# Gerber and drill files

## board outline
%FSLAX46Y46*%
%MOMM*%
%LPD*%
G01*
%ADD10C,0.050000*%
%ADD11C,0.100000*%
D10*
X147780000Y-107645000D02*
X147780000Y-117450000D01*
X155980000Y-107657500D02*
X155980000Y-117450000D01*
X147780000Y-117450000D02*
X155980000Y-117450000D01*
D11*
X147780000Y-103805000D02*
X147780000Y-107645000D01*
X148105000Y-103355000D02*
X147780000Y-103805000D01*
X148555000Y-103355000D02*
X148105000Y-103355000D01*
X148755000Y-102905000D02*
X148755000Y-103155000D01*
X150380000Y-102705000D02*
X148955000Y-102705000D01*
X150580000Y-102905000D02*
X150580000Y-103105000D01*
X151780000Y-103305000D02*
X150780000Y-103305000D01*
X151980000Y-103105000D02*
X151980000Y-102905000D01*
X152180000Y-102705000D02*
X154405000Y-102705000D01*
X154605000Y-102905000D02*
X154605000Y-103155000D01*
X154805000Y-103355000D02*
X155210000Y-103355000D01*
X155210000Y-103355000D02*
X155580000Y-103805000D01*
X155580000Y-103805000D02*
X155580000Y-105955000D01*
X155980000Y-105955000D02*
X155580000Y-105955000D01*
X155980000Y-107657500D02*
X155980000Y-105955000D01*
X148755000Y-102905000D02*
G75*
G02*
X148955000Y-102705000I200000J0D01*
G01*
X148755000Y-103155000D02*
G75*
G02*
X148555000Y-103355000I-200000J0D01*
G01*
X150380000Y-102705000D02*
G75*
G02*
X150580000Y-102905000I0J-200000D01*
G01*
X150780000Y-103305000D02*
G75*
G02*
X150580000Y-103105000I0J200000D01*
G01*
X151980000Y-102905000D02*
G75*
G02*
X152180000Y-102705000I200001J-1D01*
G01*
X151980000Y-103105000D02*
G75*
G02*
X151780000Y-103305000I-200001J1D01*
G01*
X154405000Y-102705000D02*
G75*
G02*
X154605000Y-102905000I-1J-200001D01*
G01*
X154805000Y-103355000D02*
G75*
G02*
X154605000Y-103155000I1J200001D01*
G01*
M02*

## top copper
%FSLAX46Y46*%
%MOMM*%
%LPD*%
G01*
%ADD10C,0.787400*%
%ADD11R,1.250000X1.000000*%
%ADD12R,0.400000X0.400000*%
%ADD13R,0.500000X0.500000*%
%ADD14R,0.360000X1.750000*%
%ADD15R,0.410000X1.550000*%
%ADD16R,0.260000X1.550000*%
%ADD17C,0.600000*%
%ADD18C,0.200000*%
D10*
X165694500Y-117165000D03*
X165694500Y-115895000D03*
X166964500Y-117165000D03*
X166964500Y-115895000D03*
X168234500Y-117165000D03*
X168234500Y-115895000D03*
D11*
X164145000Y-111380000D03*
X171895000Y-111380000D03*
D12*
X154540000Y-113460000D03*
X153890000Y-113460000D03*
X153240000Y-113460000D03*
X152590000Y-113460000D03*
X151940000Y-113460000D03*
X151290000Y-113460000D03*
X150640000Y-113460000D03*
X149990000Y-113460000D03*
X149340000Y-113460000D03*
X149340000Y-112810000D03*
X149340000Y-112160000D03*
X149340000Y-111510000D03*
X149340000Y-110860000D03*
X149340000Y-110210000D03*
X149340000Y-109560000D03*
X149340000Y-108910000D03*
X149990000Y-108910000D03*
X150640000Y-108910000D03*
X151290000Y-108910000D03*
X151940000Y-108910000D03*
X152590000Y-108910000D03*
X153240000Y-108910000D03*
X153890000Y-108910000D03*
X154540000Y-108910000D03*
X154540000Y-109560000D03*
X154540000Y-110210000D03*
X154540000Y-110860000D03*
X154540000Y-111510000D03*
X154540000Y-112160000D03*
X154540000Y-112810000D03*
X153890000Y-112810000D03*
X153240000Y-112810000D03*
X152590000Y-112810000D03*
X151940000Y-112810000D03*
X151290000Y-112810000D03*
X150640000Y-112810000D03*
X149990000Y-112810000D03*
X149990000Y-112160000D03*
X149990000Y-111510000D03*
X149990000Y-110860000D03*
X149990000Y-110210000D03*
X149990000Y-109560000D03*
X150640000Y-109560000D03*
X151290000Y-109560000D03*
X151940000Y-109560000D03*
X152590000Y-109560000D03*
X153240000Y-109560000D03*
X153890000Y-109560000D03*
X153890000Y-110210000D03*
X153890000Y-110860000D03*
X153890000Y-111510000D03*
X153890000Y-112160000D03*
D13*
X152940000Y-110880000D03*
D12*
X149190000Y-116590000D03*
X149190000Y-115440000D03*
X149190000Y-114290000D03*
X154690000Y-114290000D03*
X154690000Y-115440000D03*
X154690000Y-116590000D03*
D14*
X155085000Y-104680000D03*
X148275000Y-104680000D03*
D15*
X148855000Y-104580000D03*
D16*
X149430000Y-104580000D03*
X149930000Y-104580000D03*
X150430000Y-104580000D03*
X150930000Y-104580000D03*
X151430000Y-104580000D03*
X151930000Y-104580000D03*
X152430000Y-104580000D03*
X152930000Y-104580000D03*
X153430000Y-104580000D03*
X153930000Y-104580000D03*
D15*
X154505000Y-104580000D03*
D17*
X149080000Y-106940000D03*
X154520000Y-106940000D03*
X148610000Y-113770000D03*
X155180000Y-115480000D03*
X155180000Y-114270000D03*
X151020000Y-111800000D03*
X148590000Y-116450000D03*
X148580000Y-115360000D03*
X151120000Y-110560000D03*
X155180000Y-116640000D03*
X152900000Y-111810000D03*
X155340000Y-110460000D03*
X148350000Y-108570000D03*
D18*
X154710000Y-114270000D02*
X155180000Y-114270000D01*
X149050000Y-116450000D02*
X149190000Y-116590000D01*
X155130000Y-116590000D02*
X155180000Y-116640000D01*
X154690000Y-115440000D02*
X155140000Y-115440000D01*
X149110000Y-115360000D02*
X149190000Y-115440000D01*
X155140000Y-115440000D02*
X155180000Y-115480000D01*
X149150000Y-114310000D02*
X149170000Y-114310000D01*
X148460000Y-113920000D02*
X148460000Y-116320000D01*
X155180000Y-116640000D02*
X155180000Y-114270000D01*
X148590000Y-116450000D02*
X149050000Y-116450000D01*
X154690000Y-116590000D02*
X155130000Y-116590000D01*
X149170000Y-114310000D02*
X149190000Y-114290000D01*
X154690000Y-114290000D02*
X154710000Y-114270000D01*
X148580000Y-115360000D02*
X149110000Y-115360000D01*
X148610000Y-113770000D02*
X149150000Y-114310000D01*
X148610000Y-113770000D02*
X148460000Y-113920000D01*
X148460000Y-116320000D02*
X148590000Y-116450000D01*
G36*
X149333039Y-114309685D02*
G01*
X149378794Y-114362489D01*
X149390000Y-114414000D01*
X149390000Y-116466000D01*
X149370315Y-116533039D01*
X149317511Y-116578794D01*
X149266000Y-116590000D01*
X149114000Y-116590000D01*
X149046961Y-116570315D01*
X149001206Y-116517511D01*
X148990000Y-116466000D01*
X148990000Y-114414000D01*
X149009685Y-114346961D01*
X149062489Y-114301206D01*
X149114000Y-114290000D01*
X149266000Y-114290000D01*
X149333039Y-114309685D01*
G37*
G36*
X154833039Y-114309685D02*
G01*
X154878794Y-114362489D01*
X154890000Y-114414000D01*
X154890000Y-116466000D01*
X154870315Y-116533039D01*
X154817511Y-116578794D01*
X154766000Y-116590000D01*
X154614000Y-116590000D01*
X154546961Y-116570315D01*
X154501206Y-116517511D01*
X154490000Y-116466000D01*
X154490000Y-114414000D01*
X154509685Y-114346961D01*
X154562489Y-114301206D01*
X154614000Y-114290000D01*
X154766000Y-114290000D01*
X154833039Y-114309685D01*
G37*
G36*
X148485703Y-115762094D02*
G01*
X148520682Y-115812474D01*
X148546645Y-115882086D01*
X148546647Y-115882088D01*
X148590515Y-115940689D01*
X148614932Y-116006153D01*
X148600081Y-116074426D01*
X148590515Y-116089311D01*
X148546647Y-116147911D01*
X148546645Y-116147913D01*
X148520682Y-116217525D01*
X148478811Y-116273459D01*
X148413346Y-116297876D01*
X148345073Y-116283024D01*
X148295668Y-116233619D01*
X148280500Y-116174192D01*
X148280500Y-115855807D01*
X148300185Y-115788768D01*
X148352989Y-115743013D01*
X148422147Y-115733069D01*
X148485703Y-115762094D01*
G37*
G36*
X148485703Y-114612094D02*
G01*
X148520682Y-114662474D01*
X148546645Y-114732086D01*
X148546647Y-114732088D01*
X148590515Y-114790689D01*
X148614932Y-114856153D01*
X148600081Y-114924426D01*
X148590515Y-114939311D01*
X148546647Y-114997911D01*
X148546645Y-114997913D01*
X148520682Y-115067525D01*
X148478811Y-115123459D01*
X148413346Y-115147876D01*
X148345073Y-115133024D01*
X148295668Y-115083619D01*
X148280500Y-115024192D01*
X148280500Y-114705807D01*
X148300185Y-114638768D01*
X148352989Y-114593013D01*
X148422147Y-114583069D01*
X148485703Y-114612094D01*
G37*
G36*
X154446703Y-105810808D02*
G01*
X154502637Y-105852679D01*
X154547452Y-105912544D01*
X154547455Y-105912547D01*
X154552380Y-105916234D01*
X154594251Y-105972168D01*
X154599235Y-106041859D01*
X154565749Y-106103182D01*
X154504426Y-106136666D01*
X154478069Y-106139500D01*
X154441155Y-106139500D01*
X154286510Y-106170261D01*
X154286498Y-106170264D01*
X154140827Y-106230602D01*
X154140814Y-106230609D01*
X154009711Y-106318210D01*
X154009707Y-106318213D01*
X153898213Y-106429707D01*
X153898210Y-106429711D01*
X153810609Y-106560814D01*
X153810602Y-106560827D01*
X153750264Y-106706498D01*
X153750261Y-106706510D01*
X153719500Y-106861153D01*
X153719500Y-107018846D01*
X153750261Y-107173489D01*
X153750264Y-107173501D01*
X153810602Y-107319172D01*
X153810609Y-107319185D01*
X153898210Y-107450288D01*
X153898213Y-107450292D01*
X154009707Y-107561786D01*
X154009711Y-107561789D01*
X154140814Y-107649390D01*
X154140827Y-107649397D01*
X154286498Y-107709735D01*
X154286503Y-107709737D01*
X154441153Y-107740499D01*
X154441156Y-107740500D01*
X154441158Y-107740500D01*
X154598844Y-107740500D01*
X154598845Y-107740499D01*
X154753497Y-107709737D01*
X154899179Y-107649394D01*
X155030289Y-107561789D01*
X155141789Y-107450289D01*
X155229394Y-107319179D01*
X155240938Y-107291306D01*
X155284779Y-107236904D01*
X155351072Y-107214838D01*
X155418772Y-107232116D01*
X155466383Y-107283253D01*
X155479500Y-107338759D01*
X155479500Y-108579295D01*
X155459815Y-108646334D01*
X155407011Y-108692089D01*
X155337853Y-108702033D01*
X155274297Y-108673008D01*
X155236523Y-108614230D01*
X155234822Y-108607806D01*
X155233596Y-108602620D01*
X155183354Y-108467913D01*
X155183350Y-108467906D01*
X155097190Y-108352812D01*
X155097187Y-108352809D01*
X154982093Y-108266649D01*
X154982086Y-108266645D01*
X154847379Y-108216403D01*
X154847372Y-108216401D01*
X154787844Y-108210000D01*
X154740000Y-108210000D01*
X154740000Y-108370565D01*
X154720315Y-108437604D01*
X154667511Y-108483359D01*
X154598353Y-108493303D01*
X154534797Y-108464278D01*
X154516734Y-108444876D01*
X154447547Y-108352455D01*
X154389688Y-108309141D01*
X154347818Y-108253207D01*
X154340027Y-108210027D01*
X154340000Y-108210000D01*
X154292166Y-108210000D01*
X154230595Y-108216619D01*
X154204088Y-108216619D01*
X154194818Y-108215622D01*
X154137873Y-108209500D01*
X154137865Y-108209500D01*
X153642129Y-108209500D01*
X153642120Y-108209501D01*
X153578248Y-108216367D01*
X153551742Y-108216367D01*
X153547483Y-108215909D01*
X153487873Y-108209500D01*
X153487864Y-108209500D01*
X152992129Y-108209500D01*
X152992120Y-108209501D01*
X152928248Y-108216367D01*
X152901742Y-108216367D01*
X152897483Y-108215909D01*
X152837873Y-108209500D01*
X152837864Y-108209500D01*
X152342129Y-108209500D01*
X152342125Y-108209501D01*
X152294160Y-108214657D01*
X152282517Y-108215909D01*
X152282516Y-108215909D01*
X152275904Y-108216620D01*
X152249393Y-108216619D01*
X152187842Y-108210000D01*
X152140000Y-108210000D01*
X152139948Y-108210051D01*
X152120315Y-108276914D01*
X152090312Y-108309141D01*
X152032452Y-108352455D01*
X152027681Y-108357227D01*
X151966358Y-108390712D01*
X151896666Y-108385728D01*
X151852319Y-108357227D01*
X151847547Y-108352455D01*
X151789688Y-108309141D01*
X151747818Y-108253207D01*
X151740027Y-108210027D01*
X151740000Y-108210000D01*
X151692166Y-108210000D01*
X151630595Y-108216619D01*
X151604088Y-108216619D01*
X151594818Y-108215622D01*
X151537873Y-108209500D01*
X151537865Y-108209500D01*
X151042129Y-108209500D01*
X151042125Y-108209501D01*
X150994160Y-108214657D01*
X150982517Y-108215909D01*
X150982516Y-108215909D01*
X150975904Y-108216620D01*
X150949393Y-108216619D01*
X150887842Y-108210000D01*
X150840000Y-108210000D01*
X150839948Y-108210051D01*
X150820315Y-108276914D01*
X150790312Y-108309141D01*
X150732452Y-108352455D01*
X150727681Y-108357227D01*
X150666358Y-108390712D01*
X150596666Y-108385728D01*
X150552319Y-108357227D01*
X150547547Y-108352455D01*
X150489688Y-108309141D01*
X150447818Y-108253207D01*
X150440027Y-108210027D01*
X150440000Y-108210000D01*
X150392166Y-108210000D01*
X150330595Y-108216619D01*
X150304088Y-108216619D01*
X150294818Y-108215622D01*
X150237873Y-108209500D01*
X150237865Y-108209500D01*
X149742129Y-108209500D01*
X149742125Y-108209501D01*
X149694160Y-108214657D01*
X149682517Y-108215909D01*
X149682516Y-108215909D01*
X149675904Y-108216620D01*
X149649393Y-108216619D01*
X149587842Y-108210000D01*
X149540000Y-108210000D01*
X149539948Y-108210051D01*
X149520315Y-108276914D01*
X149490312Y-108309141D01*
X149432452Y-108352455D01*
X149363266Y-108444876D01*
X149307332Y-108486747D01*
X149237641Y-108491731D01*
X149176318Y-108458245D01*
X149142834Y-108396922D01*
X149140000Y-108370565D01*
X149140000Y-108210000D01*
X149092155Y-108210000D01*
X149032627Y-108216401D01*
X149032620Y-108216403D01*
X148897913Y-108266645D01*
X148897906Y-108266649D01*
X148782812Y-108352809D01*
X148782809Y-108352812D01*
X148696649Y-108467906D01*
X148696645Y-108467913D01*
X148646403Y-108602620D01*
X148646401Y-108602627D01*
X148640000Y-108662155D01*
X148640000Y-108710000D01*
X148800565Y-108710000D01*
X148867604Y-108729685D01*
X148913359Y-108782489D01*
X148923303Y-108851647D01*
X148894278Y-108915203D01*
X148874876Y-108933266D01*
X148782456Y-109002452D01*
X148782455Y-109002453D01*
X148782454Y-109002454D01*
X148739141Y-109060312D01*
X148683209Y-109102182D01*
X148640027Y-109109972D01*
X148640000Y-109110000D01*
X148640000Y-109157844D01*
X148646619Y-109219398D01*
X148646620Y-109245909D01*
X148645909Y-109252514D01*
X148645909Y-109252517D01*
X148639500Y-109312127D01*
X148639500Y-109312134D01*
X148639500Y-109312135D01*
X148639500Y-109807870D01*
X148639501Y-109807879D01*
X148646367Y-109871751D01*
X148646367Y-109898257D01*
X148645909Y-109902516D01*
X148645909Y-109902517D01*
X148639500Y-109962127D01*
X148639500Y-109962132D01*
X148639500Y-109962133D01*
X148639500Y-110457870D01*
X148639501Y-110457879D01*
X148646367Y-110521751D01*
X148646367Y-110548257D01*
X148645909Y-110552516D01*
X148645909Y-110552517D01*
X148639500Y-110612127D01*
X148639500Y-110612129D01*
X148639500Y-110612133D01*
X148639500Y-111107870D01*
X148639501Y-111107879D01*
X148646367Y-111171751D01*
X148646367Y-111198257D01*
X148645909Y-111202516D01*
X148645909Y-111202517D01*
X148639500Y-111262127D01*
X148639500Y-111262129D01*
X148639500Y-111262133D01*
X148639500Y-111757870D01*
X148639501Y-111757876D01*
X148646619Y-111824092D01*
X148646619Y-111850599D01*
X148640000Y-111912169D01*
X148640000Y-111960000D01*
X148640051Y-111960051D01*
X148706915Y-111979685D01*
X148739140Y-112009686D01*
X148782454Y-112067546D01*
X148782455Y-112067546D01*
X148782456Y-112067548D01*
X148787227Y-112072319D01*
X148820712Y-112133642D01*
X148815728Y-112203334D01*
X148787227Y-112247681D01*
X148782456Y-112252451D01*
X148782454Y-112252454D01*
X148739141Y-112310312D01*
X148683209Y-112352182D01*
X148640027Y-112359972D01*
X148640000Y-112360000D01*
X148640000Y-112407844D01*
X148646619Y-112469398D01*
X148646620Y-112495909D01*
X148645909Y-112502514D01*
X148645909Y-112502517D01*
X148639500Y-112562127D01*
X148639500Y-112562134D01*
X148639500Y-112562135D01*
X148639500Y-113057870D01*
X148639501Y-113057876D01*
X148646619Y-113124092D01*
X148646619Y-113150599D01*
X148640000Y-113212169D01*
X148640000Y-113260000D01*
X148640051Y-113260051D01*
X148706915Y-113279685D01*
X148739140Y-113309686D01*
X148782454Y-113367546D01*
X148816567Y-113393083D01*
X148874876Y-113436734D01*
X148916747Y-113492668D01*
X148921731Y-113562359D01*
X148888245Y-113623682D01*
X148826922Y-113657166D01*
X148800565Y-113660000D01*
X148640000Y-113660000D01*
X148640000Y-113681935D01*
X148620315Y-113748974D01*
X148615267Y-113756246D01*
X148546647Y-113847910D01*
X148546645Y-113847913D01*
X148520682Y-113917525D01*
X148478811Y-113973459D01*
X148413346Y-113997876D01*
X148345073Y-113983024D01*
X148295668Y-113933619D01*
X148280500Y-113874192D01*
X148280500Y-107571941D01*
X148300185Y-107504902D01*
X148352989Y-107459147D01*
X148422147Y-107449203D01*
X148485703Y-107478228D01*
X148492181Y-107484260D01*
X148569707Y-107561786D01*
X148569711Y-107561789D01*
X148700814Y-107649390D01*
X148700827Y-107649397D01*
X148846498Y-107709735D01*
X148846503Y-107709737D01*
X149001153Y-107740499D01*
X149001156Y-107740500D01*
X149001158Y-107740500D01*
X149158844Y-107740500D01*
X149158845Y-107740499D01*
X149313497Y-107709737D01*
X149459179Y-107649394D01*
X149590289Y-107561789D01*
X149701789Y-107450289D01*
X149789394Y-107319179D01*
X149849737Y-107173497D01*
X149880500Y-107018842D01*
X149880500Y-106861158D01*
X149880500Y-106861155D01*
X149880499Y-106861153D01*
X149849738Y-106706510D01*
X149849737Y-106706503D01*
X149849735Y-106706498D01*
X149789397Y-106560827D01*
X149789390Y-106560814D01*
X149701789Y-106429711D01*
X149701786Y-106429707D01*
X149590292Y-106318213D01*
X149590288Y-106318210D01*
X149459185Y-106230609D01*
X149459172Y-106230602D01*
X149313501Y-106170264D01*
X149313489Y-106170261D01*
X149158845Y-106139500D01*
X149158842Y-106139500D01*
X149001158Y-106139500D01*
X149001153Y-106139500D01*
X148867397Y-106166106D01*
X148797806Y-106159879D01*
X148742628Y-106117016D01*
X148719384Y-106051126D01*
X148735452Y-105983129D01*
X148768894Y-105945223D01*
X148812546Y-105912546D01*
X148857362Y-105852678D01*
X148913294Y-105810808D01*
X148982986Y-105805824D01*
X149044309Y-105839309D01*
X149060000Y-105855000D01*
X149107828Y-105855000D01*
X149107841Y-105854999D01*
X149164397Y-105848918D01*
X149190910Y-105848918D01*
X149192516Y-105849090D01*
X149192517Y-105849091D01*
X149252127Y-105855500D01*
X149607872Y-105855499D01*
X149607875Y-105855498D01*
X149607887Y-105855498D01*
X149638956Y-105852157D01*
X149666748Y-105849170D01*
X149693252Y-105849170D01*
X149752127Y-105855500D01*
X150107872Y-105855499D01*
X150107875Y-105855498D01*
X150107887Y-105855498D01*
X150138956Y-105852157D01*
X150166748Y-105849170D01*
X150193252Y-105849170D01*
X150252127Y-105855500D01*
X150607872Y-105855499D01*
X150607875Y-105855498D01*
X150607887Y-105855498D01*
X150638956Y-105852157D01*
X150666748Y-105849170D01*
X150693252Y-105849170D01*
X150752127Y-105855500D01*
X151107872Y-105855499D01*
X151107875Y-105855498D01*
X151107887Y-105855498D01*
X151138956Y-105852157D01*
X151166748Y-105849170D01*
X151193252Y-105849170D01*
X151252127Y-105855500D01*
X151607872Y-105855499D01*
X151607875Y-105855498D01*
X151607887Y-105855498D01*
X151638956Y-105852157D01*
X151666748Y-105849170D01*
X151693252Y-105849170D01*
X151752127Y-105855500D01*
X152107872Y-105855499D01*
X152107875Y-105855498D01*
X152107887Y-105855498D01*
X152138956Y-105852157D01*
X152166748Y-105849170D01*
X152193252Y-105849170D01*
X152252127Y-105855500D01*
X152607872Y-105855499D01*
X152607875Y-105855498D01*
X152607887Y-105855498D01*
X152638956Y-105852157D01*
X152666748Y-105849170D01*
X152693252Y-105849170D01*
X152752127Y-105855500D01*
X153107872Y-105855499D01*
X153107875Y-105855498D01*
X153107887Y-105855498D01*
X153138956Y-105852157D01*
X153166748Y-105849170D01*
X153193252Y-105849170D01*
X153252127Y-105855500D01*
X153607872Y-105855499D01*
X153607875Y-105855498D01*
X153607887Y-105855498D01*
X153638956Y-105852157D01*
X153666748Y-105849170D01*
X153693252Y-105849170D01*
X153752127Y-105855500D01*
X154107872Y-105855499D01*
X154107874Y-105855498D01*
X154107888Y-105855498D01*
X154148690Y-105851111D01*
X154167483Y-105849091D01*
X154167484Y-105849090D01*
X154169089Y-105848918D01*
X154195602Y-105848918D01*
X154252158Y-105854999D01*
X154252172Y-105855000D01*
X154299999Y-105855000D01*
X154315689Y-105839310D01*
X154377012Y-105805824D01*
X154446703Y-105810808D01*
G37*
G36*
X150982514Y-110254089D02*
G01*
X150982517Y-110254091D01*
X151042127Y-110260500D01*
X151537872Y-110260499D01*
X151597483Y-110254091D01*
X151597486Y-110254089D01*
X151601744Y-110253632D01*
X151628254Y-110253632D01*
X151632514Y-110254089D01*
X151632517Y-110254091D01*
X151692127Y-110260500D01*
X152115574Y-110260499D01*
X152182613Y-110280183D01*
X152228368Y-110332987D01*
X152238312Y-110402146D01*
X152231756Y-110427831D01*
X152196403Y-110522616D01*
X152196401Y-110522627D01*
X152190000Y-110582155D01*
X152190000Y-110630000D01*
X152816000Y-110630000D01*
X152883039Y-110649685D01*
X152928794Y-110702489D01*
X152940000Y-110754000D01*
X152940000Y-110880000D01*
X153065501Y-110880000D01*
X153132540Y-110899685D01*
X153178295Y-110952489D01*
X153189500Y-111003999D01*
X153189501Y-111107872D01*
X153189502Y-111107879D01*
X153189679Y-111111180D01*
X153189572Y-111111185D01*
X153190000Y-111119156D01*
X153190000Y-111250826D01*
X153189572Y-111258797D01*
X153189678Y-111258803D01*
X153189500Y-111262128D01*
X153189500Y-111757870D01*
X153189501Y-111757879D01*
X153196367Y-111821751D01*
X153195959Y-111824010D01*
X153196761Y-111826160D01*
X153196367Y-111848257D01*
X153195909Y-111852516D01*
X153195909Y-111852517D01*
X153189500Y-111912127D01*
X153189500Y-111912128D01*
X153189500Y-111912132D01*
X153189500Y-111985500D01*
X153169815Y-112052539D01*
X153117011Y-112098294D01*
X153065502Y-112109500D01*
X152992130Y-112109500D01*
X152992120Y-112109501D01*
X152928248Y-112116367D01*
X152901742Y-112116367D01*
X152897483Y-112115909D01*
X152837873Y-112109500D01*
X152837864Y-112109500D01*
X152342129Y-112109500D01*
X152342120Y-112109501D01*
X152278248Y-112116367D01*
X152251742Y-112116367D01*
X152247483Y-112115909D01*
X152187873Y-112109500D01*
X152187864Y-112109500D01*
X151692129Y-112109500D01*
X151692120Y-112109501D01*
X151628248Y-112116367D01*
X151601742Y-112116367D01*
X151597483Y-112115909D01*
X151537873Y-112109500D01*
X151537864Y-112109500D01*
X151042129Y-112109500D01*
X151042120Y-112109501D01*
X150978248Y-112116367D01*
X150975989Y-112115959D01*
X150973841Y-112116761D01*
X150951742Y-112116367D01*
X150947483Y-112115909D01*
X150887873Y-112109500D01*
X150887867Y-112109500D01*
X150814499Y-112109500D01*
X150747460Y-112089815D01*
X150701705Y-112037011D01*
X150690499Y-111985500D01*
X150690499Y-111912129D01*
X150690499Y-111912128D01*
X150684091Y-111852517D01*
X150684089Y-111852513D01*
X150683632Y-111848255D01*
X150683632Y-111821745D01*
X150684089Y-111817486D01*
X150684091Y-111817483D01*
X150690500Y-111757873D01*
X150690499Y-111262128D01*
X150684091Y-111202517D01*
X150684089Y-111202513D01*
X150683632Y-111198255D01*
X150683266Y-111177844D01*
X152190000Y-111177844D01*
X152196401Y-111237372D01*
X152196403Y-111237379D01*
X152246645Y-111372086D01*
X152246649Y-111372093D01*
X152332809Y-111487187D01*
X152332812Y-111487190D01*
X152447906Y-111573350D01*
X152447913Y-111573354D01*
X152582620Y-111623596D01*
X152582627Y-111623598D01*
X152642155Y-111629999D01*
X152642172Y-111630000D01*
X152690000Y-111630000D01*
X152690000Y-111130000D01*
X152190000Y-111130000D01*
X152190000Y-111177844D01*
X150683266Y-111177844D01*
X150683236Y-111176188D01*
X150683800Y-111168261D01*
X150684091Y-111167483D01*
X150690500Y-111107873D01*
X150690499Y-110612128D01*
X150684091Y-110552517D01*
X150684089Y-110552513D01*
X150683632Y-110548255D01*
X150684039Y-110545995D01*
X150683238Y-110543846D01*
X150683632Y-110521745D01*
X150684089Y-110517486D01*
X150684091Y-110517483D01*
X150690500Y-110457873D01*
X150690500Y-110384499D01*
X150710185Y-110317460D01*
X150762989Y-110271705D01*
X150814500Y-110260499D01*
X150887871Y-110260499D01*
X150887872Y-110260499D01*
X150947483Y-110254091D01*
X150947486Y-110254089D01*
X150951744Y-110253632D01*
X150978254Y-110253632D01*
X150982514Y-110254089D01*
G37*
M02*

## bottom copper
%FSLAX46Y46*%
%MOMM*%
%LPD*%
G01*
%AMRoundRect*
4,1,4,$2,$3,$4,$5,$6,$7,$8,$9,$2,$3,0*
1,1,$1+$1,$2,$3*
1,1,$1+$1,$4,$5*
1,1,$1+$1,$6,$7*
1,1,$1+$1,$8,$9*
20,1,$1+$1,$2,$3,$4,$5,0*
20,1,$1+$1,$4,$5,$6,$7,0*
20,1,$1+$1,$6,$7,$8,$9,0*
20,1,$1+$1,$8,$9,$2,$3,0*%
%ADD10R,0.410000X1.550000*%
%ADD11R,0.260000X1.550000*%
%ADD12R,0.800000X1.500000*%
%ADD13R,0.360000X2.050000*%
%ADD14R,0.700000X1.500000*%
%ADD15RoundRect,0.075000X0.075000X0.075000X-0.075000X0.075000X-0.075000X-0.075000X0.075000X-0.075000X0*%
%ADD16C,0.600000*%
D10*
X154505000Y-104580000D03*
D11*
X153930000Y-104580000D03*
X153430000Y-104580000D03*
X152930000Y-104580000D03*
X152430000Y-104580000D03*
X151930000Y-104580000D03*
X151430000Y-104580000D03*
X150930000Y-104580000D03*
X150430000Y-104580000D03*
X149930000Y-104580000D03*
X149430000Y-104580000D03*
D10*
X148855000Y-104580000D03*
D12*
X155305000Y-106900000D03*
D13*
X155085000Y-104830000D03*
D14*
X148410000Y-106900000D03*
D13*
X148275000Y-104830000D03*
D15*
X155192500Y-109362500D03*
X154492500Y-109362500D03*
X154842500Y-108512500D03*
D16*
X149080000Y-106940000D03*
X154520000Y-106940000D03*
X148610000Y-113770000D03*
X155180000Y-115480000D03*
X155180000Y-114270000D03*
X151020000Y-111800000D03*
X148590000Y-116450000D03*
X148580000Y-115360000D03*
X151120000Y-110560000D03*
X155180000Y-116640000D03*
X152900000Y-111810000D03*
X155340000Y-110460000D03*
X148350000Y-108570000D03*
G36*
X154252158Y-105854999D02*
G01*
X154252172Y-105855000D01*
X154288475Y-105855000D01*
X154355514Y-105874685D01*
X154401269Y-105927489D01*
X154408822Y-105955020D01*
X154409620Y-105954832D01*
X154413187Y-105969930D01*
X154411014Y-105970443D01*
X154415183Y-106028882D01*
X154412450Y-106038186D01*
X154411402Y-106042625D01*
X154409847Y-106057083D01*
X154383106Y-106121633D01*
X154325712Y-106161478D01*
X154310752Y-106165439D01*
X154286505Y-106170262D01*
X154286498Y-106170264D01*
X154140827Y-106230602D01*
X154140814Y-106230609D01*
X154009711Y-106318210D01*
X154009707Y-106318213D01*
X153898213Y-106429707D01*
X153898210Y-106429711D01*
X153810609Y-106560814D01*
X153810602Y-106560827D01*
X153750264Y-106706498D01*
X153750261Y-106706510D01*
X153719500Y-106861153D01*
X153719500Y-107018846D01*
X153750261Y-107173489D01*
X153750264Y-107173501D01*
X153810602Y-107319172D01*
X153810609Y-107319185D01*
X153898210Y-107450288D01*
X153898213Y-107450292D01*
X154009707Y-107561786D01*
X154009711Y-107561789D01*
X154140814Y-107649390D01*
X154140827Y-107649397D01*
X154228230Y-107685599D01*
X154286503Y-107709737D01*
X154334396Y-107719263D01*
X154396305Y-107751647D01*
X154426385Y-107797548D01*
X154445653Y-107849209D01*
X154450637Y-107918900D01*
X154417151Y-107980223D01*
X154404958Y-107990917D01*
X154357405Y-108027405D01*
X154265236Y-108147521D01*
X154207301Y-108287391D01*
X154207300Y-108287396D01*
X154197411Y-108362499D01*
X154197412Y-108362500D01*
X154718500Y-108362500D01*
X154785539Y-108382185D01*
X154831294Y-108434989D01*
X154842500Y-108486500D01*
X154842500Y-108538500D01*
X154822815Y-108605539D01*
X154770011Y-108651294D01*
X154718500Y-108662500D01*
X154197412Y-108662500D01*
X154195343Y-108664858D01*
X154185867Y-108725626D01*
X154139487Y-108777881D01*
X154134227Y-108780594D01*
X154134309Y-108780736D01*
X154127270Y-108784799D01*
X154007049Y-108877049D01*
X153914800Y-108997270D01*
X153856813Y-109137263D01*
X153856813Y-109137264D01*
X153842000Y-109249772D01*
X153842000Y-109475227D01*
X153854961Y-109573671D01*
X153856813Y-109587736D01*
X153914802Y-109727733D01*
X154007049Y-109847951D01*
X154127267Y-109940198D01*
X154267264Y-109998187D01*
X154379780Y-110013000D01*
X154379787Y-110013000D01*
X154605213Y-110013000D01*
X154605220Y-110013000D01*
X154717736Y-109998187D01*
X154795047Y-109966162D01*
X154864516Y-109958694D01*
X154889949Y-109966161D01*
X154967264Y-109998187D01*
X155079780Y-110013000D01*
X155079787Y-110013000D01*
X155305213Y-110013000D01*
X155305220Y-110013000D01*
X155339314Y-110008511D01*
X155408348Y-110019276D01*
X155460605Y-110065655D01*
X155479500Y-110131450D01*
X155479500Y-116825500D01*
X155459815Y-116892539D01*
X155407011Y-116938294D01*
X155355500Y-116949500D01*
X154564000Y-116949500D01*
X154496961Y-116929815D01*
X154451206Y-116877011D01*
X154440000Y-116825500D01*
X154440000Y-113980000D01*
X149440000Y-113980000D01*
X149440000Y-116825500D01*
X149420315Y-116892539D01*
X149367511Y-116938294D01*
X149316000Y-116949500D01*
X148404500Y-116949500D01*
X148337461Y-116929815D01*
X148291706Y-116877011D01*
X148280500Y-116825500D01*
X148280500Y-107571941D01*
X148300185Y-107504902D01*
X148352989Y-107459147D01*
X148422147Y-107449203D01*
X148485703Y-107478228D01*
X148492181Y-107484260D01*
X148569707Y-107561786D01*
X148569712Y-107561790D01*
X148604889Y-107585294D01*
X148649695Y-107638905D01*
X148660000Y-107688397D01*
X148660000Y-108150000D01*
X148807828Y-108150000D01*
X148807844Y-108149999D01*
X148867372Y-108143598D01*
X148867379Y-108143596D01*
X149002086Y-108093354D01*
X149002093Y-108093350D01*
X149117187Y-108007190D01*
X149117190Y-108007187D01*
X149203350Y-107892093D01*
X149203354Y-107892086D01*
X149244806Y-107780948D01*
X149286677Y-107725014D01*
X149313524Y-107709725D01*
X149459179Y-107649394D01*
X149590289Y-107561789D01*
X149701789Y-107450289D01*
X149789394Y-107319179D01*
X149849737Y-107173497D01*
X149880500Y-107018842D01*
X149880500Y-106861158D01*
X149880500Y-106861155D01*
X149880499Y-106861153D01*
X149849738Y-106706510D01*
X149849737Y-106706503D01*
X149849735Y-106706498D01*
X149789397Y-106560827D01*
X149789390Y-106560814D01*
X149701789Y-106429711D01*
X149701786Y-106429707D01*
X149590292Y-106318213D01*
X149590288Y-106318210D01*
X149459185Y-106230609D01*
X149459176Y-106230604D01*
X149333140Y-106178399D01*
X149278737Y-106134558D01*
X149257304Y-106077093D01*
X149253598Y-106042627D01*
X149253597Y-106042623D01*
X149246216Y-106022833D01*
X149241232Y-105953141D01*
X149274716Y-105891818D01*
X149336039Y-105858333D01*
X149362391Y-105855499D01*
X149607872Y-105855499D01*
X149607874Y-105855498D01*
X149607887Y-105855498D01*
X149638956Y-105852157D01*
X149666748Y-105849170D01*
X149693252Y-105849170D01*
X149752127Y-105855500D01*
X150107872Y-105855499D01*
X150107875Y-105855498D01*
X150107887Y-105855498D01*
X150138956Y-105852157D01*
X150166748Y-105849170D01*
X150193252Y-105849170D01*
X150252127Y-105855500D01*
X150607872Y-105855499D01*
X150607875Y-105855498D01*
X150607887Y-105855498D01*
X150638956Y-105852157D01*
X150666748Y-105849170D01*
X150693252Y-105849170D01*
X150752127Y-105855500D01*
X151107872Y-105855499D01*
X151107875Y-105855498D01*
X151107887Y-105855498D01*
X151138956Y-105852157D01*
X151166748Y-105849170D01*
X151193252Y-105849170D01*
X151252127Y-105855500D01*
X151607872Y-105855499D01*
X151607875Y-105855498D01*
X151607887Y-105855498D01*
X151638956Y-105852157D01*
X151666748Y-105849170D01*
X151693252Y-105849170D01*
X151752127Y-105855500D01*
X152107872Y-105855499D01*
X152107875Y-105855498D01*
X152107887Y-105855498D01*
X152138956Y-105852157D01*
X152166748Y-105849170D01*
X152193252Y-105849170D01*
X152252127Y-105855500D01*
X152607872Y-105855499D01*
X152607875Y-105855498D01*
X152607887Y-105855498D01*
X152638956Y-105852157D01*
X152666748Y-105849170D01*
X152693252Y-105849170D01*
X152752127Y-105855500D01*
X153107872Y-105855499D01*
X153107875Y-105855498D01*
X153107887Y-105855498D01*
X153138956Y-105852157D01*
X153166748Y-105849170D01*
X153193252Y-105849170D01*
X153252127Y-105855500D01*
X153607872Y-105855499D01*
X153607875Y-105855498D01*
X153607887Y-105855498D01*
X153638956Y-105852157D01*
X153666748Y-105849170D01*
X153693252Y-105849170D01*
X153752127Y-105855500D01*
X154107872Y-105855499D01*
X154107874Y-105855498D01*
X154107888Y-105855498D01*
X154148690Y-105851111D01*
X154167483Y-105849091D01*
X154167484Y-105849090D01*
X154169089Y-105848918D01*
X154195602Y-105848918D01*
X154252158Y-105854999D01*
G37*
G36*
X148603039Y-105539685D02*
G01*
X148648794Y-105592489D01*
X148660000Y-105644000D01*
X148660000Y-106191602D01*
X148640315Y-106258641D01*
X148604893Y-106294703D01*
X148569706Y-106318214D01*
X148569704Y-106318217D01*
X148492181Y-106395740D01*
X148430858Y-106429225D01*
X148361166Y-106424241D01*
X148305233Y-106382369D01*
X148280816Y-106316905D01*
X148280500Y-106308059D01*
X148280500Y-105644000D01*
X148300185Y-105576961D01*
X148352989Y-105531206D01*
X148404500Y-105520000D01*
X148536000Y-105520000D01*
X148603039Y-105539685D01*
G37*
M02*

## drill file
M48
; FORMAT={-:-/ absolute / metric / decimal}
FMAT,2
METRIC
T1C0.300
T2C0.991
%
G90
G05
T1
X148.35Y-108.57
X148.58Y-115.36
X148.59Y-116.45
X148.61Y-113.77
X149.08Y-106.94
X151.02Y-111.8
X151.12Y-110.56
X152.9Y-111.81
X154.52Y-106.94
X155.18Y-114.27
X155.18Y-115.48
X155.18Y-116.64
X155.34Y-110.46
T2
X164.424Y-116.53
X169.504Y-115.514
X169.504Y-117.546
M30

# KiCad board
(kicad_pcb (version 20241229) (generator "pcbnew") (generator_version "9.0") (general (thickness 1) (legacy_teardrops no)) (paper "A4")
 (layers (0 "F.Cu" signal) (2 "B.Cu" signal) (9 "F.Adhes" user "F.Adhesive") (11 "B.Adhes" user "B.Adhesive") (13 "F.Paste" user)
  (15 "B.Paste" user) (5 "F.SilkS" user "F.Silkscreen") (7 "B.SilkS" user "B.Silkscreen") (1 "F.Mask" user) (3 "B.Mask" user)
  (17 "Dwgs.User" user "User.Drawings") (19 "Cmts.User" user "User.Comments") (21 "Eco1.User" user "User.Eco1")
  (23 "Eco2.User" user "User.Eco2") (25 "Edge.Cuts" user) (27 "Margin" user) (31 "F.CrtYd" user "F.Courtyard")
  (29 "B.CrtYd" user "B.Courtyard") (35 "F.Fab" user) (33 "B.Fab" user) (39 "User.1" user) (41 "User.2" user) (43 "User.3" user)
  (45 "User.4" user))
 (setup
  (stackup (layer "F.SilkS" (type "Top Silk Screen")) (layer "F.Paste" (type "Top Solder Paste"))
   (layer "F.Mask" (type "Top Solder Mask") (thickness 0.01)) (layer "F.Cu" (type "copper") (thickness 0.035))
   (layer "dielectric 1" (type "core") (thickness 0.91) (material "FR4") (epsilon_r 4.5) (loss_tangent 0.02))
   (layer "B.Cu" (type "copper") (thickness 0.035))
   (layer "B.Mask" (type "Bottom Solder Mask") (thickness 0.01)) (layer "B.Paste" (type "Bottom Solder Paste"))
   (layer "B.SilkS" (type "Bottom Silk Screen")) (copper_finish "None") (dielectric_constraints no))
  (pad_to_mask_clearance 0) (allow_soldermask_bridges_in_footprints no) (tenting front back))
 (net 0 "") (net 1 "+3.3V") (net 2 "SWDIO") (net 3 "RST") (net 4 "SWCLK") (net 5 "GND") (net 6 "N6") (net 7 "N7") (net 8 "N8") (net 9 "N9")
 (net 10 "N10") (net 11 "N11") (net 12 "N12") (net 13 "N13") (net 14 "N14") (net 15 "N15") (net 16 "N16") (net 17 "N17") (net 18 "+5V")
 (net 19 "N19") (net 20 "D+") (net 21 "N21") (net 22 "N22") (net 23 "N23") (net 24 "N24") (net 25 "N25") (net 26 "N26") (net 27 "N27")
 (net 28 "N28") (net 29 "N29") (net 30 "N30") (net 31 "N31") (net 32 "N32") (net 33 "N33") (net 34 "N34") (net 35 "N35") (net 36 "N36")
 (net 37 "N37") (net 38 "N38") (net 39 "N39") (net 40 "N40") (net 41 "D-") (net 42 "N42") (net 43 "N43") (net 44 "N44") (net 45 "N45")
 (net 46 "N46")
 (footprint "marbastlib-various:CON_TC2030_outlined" (layer "F.Cu") (at 166.9645 116.53)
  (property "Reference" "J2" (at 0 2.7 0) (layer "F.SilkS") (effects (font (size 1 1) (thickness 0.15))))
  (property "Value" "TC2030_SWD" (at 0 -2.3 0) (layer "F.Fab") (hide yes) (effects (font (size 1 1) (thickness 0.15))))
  (pad "" np_thru_hole circle (at -2.54 0) (size 0.9906 0.9906) (drill 0.9906) (layers "*.Cu" "*.Mask"))
  (pad "" np_thru_hole circle (at 2.54 -1.016) (size 0.9906 0.9906) (drill 0.9906) (layers "*.Cu" "*.Mask"))
  (pad "" np_thru_hole circle (at 2.54 1.016) (size 0.9906 0.9906) (drill 0.9906) (layers "*.Cu" "*.Mask"))
  (pad "1" connect circle (at -1.27 0.635) (size 0.7874 0.7874) (layers "F.Cu" "F.Mask") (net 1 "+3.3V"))
  (pad "2" connect circle (at -1.27 -0.635) (size 0.7874 0.7874) (layers "F.Cu" "F.Mask") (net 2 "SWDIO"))
  (pad "3" connect circle (at 0 0.635) (size 0.7874 0.7874) (layers "F.Cu" "F.Mask") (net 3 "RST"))
  (pad "4" connect circle (at 0 -0.635) (size 0.7874 0.7874) (layers "F.Cu" "F.Mask") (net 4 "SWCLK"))
  (pad "5" connect circle (at 1.27 0.635) (size 0.7874 0.7874) (layers "F.Cu" "F.Mask") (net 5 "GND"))
  (pad "6" connect circle (at 1.27 -0.635) (size 0.7874 0.7874) (layers "F.Cu" "F.Mask") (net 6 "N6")))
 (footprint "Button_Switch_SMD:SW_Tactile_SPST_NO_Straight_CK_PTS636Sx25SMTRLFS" (layer "F.Cu") (at 168.02 111.38)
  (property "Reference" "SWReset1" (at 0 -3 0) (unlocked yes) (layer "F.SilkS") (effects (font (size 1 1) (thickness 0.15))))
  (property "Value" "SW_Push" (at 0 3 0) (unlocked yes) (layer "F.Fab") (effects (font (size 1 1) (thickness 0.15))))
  (pad "1" smd rect (at -3.875 0) (size 1.25 1) (layers "F.Cu" "F.Mask" "F.Paste") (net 5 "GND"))
  (pad "2" smd rect (at 3.875 0) (size 1.25 1) (layers "F.Cu" "F.Mask" "F.Paste") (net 3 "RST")))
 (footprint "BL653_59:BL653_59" (layer "F.Cu") (at 151.94 112.68 180)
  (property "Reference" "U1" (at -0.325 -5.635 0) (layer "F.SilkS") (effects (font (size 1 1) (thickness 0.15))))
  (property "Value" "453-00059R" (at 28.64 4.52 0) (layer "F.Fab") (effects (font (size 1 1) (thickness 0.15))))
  (pad "1" smd rect (at -2.6 -0.78 180) (size 0.4 0.4) (layers "F.Cu" "F.Mask" "F.Paste") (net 5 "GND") (solder_mask_margin 0.102))
  (pad "2" smd rect (at -1.95 -0.78 180) (size 0.4 0.4) (layers "F.Cu" "F.Mask" "F.Paste") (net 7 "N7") (solder_mask_margin 0.102))
  (pad "3" smd rect (at -1.3 -0.78 180) (size 0.4 0.4) (layers "F.Cu" "F.Mask" "F.Paste") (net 5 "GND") (solder_mask_margin 0.102))
  (pad "4" smd rect (at -0.65 -0.78 180) (size 0.4 0.4) (layers "F.Cu" "F.Mask" "F.Paste") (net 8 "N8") (solder_mask_margin 0.102))
  (pad "5" smd rect (at 0 -0.78 180) (size 0.4 0.4) (layers "F.Cu" "F.Mask" "F.Paste") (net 5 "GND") (solder_mask_margin 0.102))
  (pad "6" smd rect (at 0.65 -0.78 180) (size 0.4 0.4) (layers "F.Cu" "F.Mask" "F.Paste") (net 3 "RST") (solder_mask_margin 0.102))
  (pad "7" smd rect (at 1.3 -0.78 180) (size 0.4 0.4) (layers "F.Cu" "F.Mask" "F.Paste") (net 5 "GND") (solder_mask_margin 0.102))
  (pad "8" smd rect (at 1.95 -0.78 180) (size 0.4 0.4) (layers "F.Cu" "F.Mask" "F.Paste") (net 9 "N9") (solder_mask_margin 0.102))
  (pad "9" smd rect (at 2.6 -0.78 180) (size 0.4 0.4) (layers "F.Cu" "F.Mask" "F.Paste") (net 5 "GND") (solder_mask_margin 0.102))
  (pad "10" smd rect (at 2.6 -0.13 180) (size 0.4 0.4) (layers "F.Cu" "F.Mask" "F.Paste") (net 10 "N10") (solder_mask_margin 0.102))
  (pad "11" smd rect (at 2.6 0.52 180) (size 0.4 0.4) (layers "F.Cu" "F.Mask" "F.Paste") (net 5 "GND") (solder_mask_margin 0.102))
  (pad "12" smd rect (at 2.6 1.17 180) (size 0.4 0.4) (layers "F.Cu" "F.Mask" "F.Paste") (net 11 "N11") (solder_mask_margin 0.102))
  (pad "13" smd rect (at 2.6 1.82 180) (size 0.4 0.4) (layers "F.Cu" "F.Mask" "F.Paste") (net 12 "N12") (solder_mask_margin 0.102))
  (pad "14" smd rect (at 2.6 2.47 180) (size 0.4 0.4) (layers "F.Cu" "F.Mask" "F.Paste") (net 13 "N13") (solder_mask_margin 0.102))
  (pad "15" smd rect (at 2.6 3.12 180) (size 0.4 0.4) (layers "F.Cu" "F.Mask" "F.Paste") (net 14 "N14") (solder_mask_margin 0.102))
  (pad "16" smd rect (at 2.6 3.77 180) (size 0.4 0.4) (layers "F.Cu" "F.Mask" "F.Paste") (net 5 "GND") (solder_mask_margin 0.102))
  (pad "17" smd rect (at 1.95 3.77 180) (size 0.4 0.4) (layers "F.Cu" "F.Mask" "F.Paste") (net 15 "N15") (solder_mask_margin 0.102))
  (pad "18" smd rect (at 1.3 3.77 180) (size 0.4 0.4) (layers "F.Cu" "F.Mask" "F.Paste") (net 5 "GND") (solder_mask_margin 0.102))
  (pad "19" smd rect (at 0.65 3.77 180) (size 0.4 0.4) (layers "F.Cu" "F.Mask" "F.Paste") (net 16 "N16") (solder_mask_margin 0.102))
  (pad "20" smd rect (at 0 3.77 180) (size 0.4 0.4) (layers "F.Cu" "F.Mask" "F.Paste") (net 5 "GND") (solder_mask_margin 0.102))
  (pad "21" smd rect (at -0.65 3.77 180) (size 0.4 0.4) (layers "F.Cu" "F.Mask" "F.Paste") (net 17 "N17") (solder_mask_margin 0.102))
  (pad "22" smd rect (at -1.3 3.77 180) (size 0.4 0.4) (layers "F.Cu" "F.Mask" "F.Paste") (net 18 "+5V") (solder_mask_margin 0.102))
  (pad "23" smd rect (at -1.95 3.77 180) (size 0.4 0.4) (layers "F.Cu" "F.Mask" "F.Paste") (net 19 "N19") (solder_mask_margin 0.102))
  (pad "24" smd rect (at -2.6 3.77 180) (size 0.4 0.4) (layers "F.Cu" "F.Mask" "F.Paste") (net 5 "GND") (solder_mask_margin 0.102))
  (pad "25" smd rect (at -2.6 3.12 180) (size 0.4 0.4) (layers "F.Cu" "F.Mask" "F.Paste") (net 18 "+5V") (solder_mask_margin 0.102))
  (pad "26" smd rect (at -2.6 2.47 180) (size 0.4 0.4) (layers "F.Cu" "F.Mask" "F.Paste") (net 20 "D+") (solder_mask_margin 0.102))
  (pad "27" smd rect (at -2.6 1.82 180) (size 0.4 0.4) (layers "F.Cu" "F.Mask" "F.Paste") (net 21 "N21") (solder_mask_margin 0.102))
  (pad "28" smd rect (at -2.6 1.17 180) (size 0.4 0.4) (layers "F.Cu" "F.Mask" "F.Paste") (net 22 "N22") (solder_mask_margin 0.102))
  (pad "29" smd rect (at -2.6 0.52 180) (size 0.4 0.4) (layers "F.Cu" "F.Mask" "F.Paste") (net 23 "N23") (solder_mask_margin 0.102))
  (pad "30" smd rect (at -2.6 -0.13 180) (size 0.4 0.4) (layers "F.Cu" "F.Mask" "F.Paste") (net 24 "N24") (solder_mask_margin 0.102))
  (pad "31" smd rect (at -1.95 -0.13 180) (size 0.4 0.4) (layers "F.Cu" "F.Mask" "F.Paste") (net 4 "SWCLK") (solder_mask_margin 0.102))
  (pad "32" smd rect (at -1.3 -0.13 180) (size 0.4 0.4) (layers "F.Cu" "F.Mask" "F.Paste") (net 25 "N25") (solder_mask_margin 0.102))
  (pad "33" smd rect (at -0.65 -0.13 180) (size 0.4 0.4) (layers "F.Cu" "F.Mask" "F.Paste") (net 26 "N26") (solder_mask_margin 0.102))
  (pad "34" smd rect (at 0 -0.13 180) (size 0.4 0.4) (layers "F.Cu" "F.Mask" "F.Paste") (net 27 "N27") (solder_mask_margin 0.102))
  (pad "35" smd rect (at 0.65 -0.13 180) (size 0.4 0.4) (layers "F.Cu" "F.Mask" "F.Paste") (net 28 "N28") (solder_mask_margin 0.102))
  (pad "36" smd rect (at 1.3 -0.13 180) (size 0.4 0.4) (layers "F.Cu" "F.Mask" "F.Paste") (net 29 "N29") (solder_mask_margin 0.102))
  (pad "37" smd rect (at 1.95 -0.13 180) (size 0.4 0.4) (layers "F.Cu" "F.Mask" "F.Paste") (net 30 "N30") (solder_mask_margin 0.102))
  (pad "38" smd rect (at 1.95 0.52 180) (size 0.4 0.4) (layers "F.Cu" "F.Mask" "F.Paste") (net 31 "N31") (solder_mask_margin 0.102))
  (pad "39" smd rect (at 1.95 1.17 180) (size 0.4 0.4) (layers "F.Cu" "F.Mask" "F.Paste") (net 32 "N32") (solder_mask_margin 0.102))
  (pad "40" smd rect (at 1.95 1.82 180) (size 0.4 0.4) (layers "F.Cu" "F.Mask" "F.Paste") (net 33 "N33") (solder_mask_margin 0.102))
  (pad "41" smd rect (at 1.95 2.47 180) (size 0.4 0.4) (layers "F.Cu" "F.Mask" "F.Paste") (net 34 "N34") (solder_mask_margin 0.102))
  (pad "42" smd rect (at 1.95 3.12 180) (size 0.4 0.4) (layers "F.Cu" "F.Mask" "F.Paste") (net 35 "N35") (solder_mask_margin 0.102))
  (pad "43" smd rect (at 1.3 3.12 180) (size 0.4 0.4) (layers "F.Cu" "F.Mask" "F.Paste") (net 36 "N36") (solder_mask_margin 0.102))
  (pad "44" smd rect (at 0.65 3.12 180) (size 0.4 0.4) (layers "F.Cu" "F.Mask" "F.Paste") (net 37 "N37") (solder_mask_margin 0.102))
  (pad "45" smd rect (at 0 3.12 180) (size 0.4 0.4) (layers "F.Cu" "F.Mask" "F.Paste") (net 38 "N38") (solder_mask_margin 0.102))
  (pad "46" smd rect (at -0.65 3.12 180) (size 0.4 0.4) (layers "F.Cu" "F.Mask" "F.Paste") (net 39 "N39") (solder_mask_margin 0.102))
  (pad "47" smd rect (at -1.3 3.12 180) (size 0.4 0.4) (layers "F.Cu" "F.Mask" "F.Paste") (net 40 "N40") (solder_mask_margin 0.102))
  (pad "48" smd rect (at -1.95 3.12 180) (size 0.4 0.4) (layers "F.Cu" "F.Mask" "F.Paste") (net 5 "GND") (solder_mask_margin 0.102))
  (pad "49" smd rect (at -1.95 2.47 180) (size 0.4 0.4) (layers "F.Cu" "F.Mask" "F.Paste") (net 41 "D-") (solder_mask_margin 0.102))
  (pad "50" smd rect (at -1.95 1.82 180) (size 0.4 0.4) (layers "F.Cu" "F.Mask" "F.Paste") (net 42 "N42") (solder_mask_margin 0.102))
  (pad "51" smd rect (at -1.95 1.17 180) (size 0.4 0.4) (layers "F.Cu" "F.Mask" "F.Paste") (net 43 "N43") (solder_mask_margin 0.102))
  (pad "52" smd rect (at -1.95 0.52 180) (size 0.4 0.4) (layers "F.Cu" "F.Mask" "F.Paste") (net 2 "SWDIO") (solder_mask_margin 0.102))
  (pad "G1" smd rect (at -1 1.8 180) (size 0.5 0.5) (layers "F.Cu" "F.Mask" "F.Paste") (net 5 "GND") (solder_mask_margin 0.102))
  (pad "G2" smd rect (at 2.75 -3.91 180) (size 0.4 0.4) (layers "F.Cu" "F.Mask" "F.Paste") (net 5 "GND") (solder_mask_margin 0.102))
  (pad "G3" smd rect (at 2.75 -2.76 180) (size 0.4 0.4) (layers "F.Cu" "F.Mask" "F.Paste") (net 5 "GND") (solder_mask_margin 0.102))
  (pad "G4" smd rect (at 2.75 -1.61 180) (size 0.4 0.4) (layers "F.Cu" "F.Mask" "F.Paste") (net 5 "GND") (solder_mask_margin 0.102))
  (pad "G5" smd rect (at -2.75 -1.61 180) (size 0.4 0.4) (layers "F.Cu" "F.Mask" "F.Paste") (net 5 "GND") (solder_mask_margin 0.102))
  (pad "G6" smd rect (at -2.75 -2.76 180) (size 0.4 0.4) (layers "F.Cu" "F.Mask" "F.Paste") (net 5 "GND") (solder_mask_margin 0.102))
  (pad "G7" smd rect (at -2.75 -3.91 180) (size 0.4 0.4) (layers "F.Cu" "F.Mask" "F.Paste") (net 5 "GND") (solder_mask_margin 0.102))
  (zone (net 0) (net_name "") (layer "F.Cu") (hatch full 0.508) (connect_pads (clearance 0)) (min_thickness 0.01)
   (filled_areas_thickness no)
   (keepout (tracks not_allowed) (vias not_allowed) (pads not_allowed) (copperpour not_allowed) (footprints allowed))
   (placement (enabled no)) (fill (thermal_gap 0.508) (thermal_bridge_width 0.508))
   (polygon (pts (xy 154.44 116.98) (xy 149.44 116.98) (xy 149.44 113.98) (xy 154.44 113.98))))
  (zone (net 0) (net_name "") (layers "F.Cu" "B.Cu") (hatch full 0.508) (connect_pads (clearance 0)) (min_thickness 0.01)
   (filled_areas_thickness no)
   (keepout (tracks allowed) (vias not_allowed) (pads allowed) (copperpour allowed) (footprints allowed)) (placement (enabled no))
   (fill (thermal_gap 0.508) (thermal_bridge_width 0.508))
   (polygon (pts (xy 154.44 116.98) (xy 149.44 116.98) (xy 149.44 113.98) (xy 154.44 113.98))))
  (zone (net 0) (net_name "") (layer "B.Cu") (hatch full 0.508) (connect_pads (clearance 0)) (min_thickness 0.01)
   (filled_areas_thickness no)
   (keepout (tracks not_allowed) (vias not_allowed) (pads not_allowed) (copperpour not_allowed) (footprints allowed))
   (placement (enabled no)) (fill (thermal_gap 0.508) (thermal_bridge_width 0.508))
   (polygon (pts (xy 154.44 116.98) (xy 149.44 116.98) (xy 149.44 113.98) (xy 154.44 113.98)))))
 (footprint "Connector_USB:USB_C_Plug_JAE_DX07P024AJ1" (layer "F.Cu") (at 151.68 105.7275 180)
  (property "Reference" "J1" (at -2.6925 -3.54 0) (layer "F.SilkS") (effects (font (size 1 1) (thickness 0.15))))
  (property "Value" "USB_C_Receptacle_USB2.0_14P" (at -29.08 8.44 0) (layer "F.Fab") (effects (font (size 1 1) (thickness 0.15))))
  (fp_line (start 3.9 1.9225) (end 3.9 -1.9175) (stroke (width 0.1) (type solid)) (layer "Edge.Cuts"))
  (fp_line (start 3.575 2.3725) (end 3.9 1.9225) (stroke (width 0.1) (type solid)) (layer "Edge.Cuts"))
  (fp_line (start 3.125 2.3725) (end 3.575 2.3725) (stroke (width 0.1) (type solid)) (layer "Edge.Cuts"))
  (fp_line (start 2.925 2.8225) (end 2.925 2.5725) (stroke (width 0.1) (type solid)) (layer "Edge.Cuts"))
  (fp_line (start 1.3 3.0225) (end 2.725 3.0225) (stroke (width 0.1) (type solid)) (layer "Edge.Cuts"))
  (fp_line (start 1.1 2.8225) (end 1.1 2.6225) (stroke (width 0.1) (type solid)) (layer "Edge.Cuts"))
  (fp_line (start -0.1 2.4225) (end 0.9 2.4225) (stroke (width 0.1) (type solid)) (layer "Edge.Cuts"))
  (fp_line (start -0.3 2.6225) (end -0.3 2.8225) (stroke (width 0.1) (type solid)) (layer "Edge.Cuts"))
  (fp_line (start -0.5 3.0225) (end -2.725 3.0225) (stroke (width 0.1) (type solid)) (layer "Edge.Cuts"))
  (fp_line (start -2.925 2.8225) (end -2.925 2.5725) (stroke (width 0.1) (type solid)) (layer "Edge.Cuts"))
  (fp_line (start -3.125 2.3725) (end -3.53 2.3725) (stroke (width 0.1) (type solid)) (layer "Edge.Cuts"))
  (fp_line (start -3.53 2.3725) (end -3.9 1.9225) (stroke (width 0.1) (type solid)) (layer "Edge.Cuts"))
  (fp_line (start -3.9 1.9225) (end -3.9 -0.2275) (stroke (width 0.1) (type solid)) (layer "Edge.Cuts"))
  (fp_line (start -4.3 -0.2275) (end -3.9 -0.2275) (stroke (width 0.1) (type solid)) (layer "Edge.Cuts"))
  (fp_line (start -4.3 -1.93) (end -4.3 -0.2275) (stroke (width 0.1) (type solid)) (layer "Edge.Cuts"))
  (fp_arc (start 2.925 2.8225) (mid 2.866421 2.963921) (end 2.725 3.0225) (stroke (width 0.1) (type solid)) (layer "Edge.Cuts"))
  (fp_arc (start 2.925 2.5725) (mid 2.983579 2.431079) (end 3.125 2.3725) (stroke (width 0.1) (type solid)) (layer "Edge.Cuts"))
  (fp_arc (start 1.3 3.0225) (mid 1.158579 2.963921) (end 1.1 2.8225) (stroke (width 0.1) (type solid)) (layer "Edge.Cuts"))
  (fp_arc (start 0.9 2.4225) (mid 1.041421 2.481079) (end 1.1 2.6225) (stroke (width 0.1) (type solid)) (layer "Edge.Cuts"))
  (fp_arc (start -0.3 2.8225) (mid -0.358579 2.963921) (end -0.5 3.0225) (stroke (width 0.1) (type solid)) (layer "Edge.Cuts"))
  (fp_arc (start -0.3 2.6225) (mid -0.241421 2.481079) (end -0.1 2.4225) (stroke (width 0.1) (type solid)) (layer "Edge.Cuts"))
  (fp_arc (start -2.725 3.0225) (mid -2.866421 2.963921) (end -2.925 2.8225) (stroke (width 0.1) (type solid)) (layer "Edge.Cuts"))
  (fp_arc (start -3.125 2.3725) (mid -2.983579 2.431079) (end -2.925 2.5725) (stroke (width 0.1) (type solid)) (layer "Edge.Cuts"))
  (pad "" smd rect (at -3.405 1.0475 180) (size 0.36 1.75) (layers "F.Cu" "F.Mask"))
  (pad "" smd rect (at 3.405 1.0475 180) (size 0.36 1.75) (layers "F.Cu" "F.Mask"))
  (pad "A1" smd rect (at 2.825 1.1475 180) (size 0.41 1.55) (layers "F.Cu" "F.Mask" "F.Paste") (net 5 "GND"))
  (pad "A2" smd rect (at 2.25 1.1475 180) (size 0.26 1.55) (layers "F.Cu" "F.Mask" "F.Paste"))
  (pad "A3" smd rect (at 1.75 1.1475 180) (size 0.26 1.55) (layers "F.Cu" "F.Mask" "F.Paste"))
  (pad "A4" smd rect (at 1.25 1.1475 180) (size 0.26 1.55) (layers "F.Cu" "F.Mask" "F.Paste") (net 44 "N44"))
  (pad "A5" smd rect (at 0.75 1.1475 180) (size 0.26 1.55) (layers "F.Cu" "F.Mask" "F.Paste") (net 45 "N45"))
  (pad "A6" smd rect (at 0.25 1.1475) (size 0.26 1.55) (layers "F.Cu" "F.Mask" "F.Paste") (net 20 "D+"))
  (pad "A7" smd rect (at -0.25 1.1475) (size 0.26 1.55) (layers "F.Cu" "F.Mask" "F.Paste") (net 41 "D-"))
  (pad "A8" smd rect (at -0.75 1.1475 180) (size 0.26 1.55) (layers "F.Cu" "F.Mask" "F.Paste"))
  (pad "A9" smd rect (at -1.25 1.1475 180) (size 0.26 1.55) (layers "F.Cu" "F.Mask" "F.Paste") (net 44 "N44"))
  (pad "A10" smd rect (at -1.75 1.1475 180) (size 0.26 1.55) (layers "F.Cu" "F.Mask" "F.Paste"))
  (pad "A11" smd rect (at -2.25 1.1475 180) (size 0.26 1.55) (layers "F.Cu" "F.Mask" "F.Paste"))
  (pad "A12" smd rect (at -2.825 1.1475 180) (size 0.41 1.55) (layers "F.Cu" "F.Mask" "F.Paste") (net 5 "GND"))
  (pad "B1" smd rect (at -2.825 1.1475 180) (size 0.41 1.55) (layers "B.Cu" "B.Mask" "B.Paste") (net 5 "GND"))
  (pad "B2" smd rect (at -2.25 1.1475 180) (size 0.26 1.55) (layers "B.Cu" "B.Mask" "B.Paste"))
  (pad "B3" smd rect (at -1.75 1.1475 180) (size 0.26 1.55) (layers "B.Cu" "B.Mask" "B.Paste"))
  (pad "B4" smd rect (at -1.25 1.1475 180) (size 0.26 1.55) (layers "B.Cu" "B.Mask" "B.Paste") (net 44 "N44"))
  (pad "B5" smd rect (at -0.75 1.1475 180) (size 0.26 1.55) (layers "B.Cu" "B.Mask" "B.Paste") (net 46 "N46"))
  (pad "B6" smd rect (at -0.25 1.1475) (size 0.26 1.55) (layers "B.Cu" "B.Mask" "B.Paste") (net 20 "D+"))
  (pad "B7" smd rect (at 0.25 1.1475 180) (size 0.26 1.55) (layers "B.Cu" "B.Mask" "B.Paste") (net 41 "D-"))
  (pad "B8" smd rect (at 0.75 1.1475 180) (size 0.26 1.55) (layers "B.Cu" "B.Mask" "B.Paste"))
  (pad "B9" smd rect (at 1.25 1.1475 180) (size 0.26 1.55) (layers "B.Cu" "B.Mask" "B.Paste") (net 44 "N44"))
  (pad "B10" smd rect (at 1.75 1.1475 180) (size 0.26 1.55) (layers "B.Cu" "B.Mask" "B.Paste"))
  (pad "B11" smd rect (at 2.25 1.1475 180) (size 0.26 1.55) (layers "B.Cu" "B.Mask" "B.Paste"))
  (pad "B12" smd rect (at 2.825 1.1475 180) (size 0.41 1.55) (layers "B.Cu" "B.Mask" "B.Paste") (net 5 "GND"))
  (pad "S1" smd rect (at -3.625 -1.1725 180) (size 0.8 1.5) (layers "B.Cu" "B.Mask" "B.Paste") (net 5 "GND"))
  (pad "S1" smd rect (at -3.405 0.8975 180) (size 0.36 2.05) (layers "B.Cu" "B.Mask" "B.Paste") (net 5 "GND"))
  (pad "S1" smd rect (at 3.27 -1.1725) (size 0.7 1.5) (layers "B.Cu" "B.Mask" "B.Paste") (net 5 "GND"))
  (pad "S1" smd rect (at 3.405 0.8975 180) (size 0.36 2.05) (layers "B.Cu" "B.Mask" "B.Paste") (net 5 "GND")))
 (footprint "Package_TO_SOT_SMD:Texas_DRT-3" (layer "B.Cu") (at 154.8425 108.9375 180)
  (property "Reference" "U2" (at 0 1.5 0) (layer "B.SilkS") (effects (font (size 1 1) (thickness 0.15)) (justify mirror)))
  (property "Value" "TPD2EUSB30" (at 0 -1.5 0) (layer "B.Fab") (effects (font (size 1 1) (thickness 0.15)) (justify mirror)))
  (pad "1" smd roundrect (at -0.35 -0.425 180) (size 0.3 0.3) (layers "B.Cu" "B.Mask" "B.Paste") (roundrect_rratio 0.25) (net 20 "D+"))
  (pad "2" smd roundrect (at 0.35 -0.425 180) (size 0.3 0.3) (layers "B.Cu" "B.Mask" "B.Paste") (roundrect_rratio 0.25) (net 41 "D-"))
  (pad "3" smd roundrect (at 0 0.425 180) (size 0.3 0.3) (layers "B.Cu" "B.Mask" "B.Paste") (roundrect_rratio 0.25) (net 5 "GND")))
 (gr_line (start 147.78 107.645) (end 147.78 117.45) (stroke (width 0.05) (type default)) (layer "Edge.Cuts"))
 (gr_line (start 155.98 107.6575) (end 155.98 117.45) (stroke (width 0.05) (type default)) (layer "Edge.Cuts"))
 (gr_line (start 147.78 117.45) (end 155.98 117.45) (stroke (width 0.05) (type default)) (layer "Edge.Cuts"))
 (via (at 149.08 106.94) (size 0.6) (drill 0.3) (layers "F.Cu" "B.Cu") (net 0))
 (via (at 154.52 106.94) (size 0.6) (drill 0.3) (layers "F.Cu" "B.Cu") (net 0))
 (segment (start 154.71 114.27) (end 155.18 114.27) (width 0.2) (layer "F.Cu") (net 5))
 (segment (start 149.05 116.45) (end 149.19 116.59) (width 0.2) (layer "F.Cu") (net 5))
 (segment (start 155.13 116.59) (end 155.18 116.64) (width 0.2) (layer "F.Cu") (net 5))
 (segment (start 154.69 115.44) (end 155.14 115.44) (width 0.2) (layer "F.Cu") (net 5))
 (segment (start 149.11 115.36) (end 149.19 115.44) (width 0.2) (layer "F.Cu") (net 5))
 (segment (start 155.14 115.44) (end 155.18 115.48) (width 0.2) (layer "F.Cu") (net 5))
 (segment (start 149.15 114.31) (end 149.17 114.31) (width 0.2) (layer "F.Cu") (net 5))
 (segment (start 148.46 113.92) (end 148.46 116.32) (width 0.2) (layer "F.Cu") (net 5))
 (segment (start 155.18 116.64) (end 155.18 114.27) (width 0.2) (layer "F.Cu") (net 5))
 (segment (start 148.59 116.45) (end 149.05 116.45) (width 0.2) (layer "F.Cu") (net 5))
 (segment (start 154.69 116.59) (end 155.13 116.59) (width 0.2) (layer "F.Cu") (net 5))
 (segment (start 149.17 114.31) (end 149.19 114.29) (width 0.2) (layer "F.Cu") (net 5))
 (segment (start 154.69 114.29) (end 154.71 114.27) (width 0.2) (layer "F.Cu") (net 5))
 (segment (start 148.58 115.36) (end 149.11 115.36) (width 0.2) (layer "F.Cu") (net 5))
 (segment (start 148.61 113.77) (end 149.15 114.31) (width 0.2) (layer "F.Cu") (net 5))
 (segment (start 148.61 113.77) (end 148.46 113.92) (width 0.2) (layer "F.Cu") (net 5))
 (segment (start 148.46 116.32) (end 148.59 116.45) (width 0.2) (layer "F.Cu") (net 5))
 (via (at 148.61 113.77) (size 0.6) (drill 0.3) (layers "F.Cu" "B.Cu") (free yes) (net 5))
 (via (at 155.18 115.48) (size 0.6) (drill 0.3) (layers "F.Cu" "B.Cu") (free yes) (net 5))
 (via (at 155.18 114.27) (size 0.6) (drill 0.3) (layers "F.Cu" "B.Cu") (free yes) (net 5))
 (via (at 151.02 111.8) (size 0.6) (drill 0.3) (layers "F.Cu" "B.Cu") (free yes) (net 5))
 (via (at 148.59 116.45) (size 0.6) (drill 0.3) (layers "F.Cu" "B.Cu") (free yes) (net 5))
 (via (at 148.58 115.36) (size 0.6) (drill 0.3) (layers "F.Cu" "B.Cu") (free yes) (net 5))
 (via (at 151.12 110.56) (size 0.6) (drill 0.3) (layers "F.Cu" "B.Cu") (free yes) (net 5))
 (via (at 155.18 116.64) (size 0.6) (drill 0.3) (layers "F.Cu" "B.Cu") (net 5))
 (via (at 152.9 111.81) (size 0.6) (drill 0.3) (layers "F.Cu" "B.Cu") (free yes) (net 5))
 (via (at 155.34 110.46) (size 0.6) (drill 0.3) (layers "F.Cu" "B.Cu") (free yes) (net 5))
 (via (at 148.35 108.57) (size 0.6) (drill 0.3) (layers "F.Cu" "B.Cu") (free yes) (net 5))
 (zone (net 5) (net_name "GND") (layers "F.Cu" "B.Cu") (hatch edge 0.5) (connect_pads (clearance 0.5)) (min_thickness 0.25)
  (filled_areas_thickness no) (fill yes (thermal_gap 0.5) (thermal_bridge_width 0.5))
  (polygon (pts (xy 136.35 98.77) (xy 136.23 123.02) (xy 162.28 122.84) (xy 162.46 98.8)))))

